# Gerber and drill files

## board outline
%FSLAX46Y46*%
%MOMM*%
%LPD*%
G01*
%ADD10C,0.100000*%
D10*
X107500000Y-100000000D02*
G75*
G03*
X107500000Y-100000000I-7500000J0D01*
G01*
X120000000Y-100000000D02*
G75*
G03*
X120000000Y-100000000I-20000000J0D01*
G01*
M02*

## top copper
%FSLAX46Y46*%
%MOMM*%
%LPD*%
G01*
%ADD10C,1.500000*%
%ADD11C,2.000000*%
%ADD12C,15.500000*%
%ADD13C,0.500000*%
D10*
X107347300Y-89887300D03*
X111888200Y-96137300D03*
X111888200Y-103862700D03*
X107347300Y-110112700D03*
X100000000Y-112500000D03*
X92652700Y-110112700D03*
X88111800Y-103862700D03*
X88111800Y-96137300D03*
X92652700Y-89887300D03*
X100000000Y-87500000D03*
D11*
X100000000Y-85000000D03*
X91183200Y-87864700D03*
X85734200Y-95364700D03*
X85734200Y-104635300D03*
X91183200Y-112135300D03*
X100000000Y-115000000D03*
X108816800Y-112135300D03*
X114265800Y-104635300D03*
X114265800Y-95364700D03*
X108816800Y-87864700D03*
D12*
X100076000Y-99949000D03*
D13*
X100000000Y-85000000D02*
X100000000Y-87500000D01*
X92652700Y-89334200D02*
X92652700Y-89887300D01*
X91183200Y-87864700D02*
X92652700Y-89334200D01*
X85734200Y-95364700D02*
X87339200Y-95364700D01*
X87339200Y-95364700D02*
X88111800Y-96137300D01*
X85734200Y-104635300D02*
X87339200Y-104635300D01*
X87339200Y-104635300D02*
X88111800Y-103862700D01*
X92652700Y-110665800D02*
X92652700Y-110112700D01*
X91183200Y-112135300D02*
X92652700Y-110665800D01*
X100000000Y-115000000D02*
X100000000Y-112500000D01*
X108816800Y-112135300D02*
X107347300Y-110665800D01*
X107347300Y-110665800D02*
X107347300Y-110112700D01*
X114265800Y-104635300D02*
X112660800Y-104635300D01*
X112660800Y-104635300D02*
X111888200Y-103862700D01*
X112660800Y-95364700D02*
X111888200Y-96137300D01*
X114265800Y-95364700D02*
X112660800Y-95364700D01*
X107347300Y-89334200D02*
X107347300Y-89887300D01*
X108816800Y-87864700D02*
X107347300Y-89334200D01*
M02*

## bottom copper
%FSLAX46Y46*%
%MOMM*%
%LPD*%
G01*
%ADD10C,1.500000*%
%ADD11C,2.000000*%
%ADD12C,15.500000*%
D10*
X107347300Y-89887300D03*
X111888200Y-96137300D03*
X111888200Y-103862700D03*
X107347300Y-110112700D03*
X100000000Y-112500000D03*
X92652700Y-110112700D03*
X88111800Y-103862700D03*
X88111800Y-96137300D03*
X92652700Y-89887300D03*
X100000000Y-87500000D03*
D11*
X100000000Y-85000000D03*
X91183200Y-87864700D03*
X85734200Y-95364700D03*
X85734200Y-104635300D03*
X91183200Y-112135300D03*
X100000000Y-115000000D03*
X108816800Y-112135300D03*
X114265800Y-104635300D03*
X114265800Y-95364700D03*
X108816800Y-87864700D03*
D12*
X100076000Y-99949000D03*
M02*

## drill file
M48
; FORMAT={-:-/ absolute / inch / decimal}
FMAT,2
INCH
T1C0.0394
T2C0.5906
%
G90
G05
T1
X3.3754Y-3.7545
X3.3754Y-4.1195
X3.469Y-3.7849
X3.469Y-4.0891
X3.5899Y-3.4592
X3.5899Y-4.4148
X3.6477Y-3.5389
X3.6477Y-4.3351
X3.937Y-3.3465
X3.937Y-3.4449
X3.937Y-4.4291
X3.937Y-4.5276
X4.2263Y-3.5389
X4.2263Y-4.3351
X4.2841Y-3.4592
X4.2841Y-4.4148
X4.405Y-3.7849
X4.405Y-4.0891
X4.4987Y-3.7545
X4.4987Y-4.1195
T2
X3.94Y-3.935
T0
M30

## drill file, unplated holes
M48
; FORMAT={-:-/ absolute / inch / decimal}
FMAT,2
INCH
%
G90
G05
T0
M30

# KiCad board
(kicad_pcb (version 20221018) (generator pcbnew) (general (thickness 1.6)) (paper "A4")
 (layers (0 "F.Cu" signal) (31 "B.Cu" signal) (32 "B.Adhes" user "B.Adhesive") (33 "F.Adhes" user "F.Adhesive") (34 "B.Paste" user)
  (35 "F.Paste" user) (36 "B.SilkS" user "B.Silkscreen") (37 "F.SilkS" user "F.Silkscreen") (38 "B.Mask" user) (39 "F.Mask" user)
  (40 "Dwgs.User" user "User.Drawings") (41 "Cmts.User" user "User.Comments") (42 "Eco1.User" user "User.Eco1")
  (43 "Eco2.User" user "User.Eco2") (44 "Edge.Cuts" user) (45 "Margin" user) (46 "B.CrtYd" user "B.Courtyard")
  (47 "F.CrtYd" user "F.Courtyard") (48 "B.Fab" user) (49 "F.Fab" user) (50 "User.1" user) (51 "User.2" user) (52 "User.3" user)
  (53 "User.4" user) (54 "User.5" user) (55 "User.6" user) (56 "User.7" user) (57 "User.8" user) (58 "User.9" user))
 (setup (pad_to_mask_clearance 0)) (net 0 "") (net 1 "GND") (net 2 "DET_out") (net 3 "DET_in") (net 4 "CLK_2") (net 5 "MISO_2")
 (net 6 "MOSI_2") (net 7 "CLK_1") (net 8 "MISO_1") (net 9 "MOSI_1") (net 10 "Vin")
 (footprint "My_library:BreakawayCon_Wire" (layer "B.Cu") (at 100 100)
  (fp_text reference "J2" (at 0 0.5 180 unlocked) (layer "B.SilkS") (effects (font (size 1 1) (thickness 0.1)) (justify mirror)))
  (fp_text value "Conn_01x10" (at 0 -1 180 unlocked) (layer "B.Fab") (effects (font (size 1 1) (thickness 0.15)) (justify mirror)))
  (pad "1" thru_hole circle (at 0 -12.5) (size 1.5 1.5) (drill 1) (layers "*.Cu" "*.Mask") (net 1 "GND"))
  (pad "2" thru_hole circle (at -7.3473 -10.1127) (size 1.5 1.5) (drill 1) (layers "*.Cu" "*.Mask") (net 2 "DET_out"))
  (pad "3" thru_hole circle (at -11.8882 -3.8627) (size 1.5 1.5) (drill 1) (layers "*.Cu" "*.Mask") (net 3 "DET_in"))
  (pad "4" thru_hole circle (at -11.8882 3.8627) (size 1.5 1.5) (drill 1) (layers "*.Cu" "*.Mask") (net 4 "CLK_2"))
  (pad "5" thru_hole circle (at -7.3473 10.1127) (size 1.5 1.5) (drill 1) (layers "*.Cu" "*.Mask") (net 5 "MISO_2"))
  (pad "6" thru_hole circle (at 0 12.5) (size 1.5 1.5) (drill 1) (layers "*.Cu" "*.Mask") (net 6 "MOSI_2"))
  (pad "7" thru_hole circle (at 7.3473 10.1127) (size 1.5 1.5) (drill 1) (layers "*.Cu" "*.Mask") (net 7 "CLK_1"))
  (pad "8" thru_hole circle (at 11.8882 3.8627) (size 1.5 1.5) (drill 1) (layers "*.Cu" "*.Mask") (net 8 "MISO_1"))
  (pad "9" thru_hole circle (at 11.8882 -3.8627) (size 1.5 1.5) (drill 1) (layers "*.Cu" "*.Mask") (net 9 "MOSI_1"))
  (pad "10" thru_hole circle (at 7.3473 -10.1127) (size 1.5 1.5) (drill 1) (layers "*.Cu" "*.Mask") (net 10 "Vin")))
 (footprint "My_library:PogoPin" (layer "B.Cu") (at 100 100)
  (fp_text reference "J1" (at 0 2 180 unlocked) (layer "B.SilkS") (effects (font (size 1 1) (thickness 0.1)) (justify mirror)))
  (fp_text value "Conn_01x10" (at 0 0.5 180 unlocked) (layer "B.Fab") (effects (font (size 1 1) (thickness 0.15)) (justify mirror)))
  (pad "1" thru_hole circle (at 0 -15) (size 2 2) (drill 1) (layers "*.Cu" "*.Mask") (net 1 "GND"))
  (pad "2" thru_hole circle (at -8.8168 -12.1353) (size 2 2) (drill 1) (layers "*.Cu" "*.Mask") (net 2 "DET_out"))
  (pad "3" thru_hole circle (at -14.2658 -4.6353) (size 2 2) (drill 1) (layers "*.Cu" "*.Mask") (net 3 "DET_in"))
  (pad "4" thru_hole circle (at -14.2658 4.6353) (size 2 2) (drill 1) (layers "*.Cu" "*.Mask") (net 4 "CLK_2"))
  (pad "5" thru_hole circle (at -8.8168 12.1353) (size 2 2) (drill 1) (layers "*.Cu" "*.Mask") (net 5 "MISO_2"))
  (pad "6" thru_hole circle (at 0 15) (size 2 2) (drill 1) (layers "*.Cu" "*.Mask") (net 6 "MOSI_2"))
  (pad "7" thru_hole circle (at 8.8168 12.1353) (size 2 2) (drill 1) (layers "*.Cu" "*.Mask") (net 7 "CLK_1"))
  (pad "8" thru_hole circle (at 14.2658 4.6353) (size 2 2) (drill 1) (layers "*.Cu" "*.Mask") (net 8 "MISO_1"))
  (pad "9" thru_hole circle (at 14.2658 -4.6353) (size 2 2) (drill 1) (layers "*.Cu" "*.Mask") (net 9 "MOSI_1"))
  (pad "10" thru_hole circle (at 8.8168 -12.1353) (size 2 2) (drill 1) (layers "*.Cu" "*.Mask") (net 10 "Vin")))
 (gr_circle (center 100 100) (end 107.5 100) (stroke (width 0.1) (type default)) (fill none) (layer "Edge.Cuts"))
 (gr_circle (center 100 100) (end 120 100) (stroke (width 0.1) (type default)) (fill none) (layer "Edge.Cuts"))
 (via (at 100.076 99.949) (size 15.5) (drill 15) (layers "F.Cu" "B.Cu") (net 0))
 (segment (start 100 85) (end 100 87.5) (width 0.5) (layer "F.Cu") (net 1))
 (segment (start 92.6527 89.3342) (end 92.6527 89.8873) (width 0.5) (layer "F.Cu") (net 2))
 (segment (start 91.1832 87.8647) (end 92.6527 89.3342) (width 0.5) (layer "F.Cu") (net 2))
 (segment (start 85.7342 95.3647) (end 87.3392 95.3647) (width 0.5) (layer "F.Cu") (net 3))
 (segment (start 87.3392 95.3647) (end 88.1118 96.1373) (width 0.5) (layer "F.Cu") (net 3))
 (segment (start 85.7342 104.6353) (end 87.3392 104.6353) (width 0.5) (layer "F.Cu") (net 4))
 (segment (start 87.3392 104.6353) (end 88.1118 103.8627) (width 0.5) (layer "F.Cu") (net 4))
 (segment (start 92.6527 110.6658) (end 92.6527 110.1127) (width 0.5) (layer "F.Cu") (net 5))
 (segment (start 91.1832 112.1353) (end 92.6527 110.6658) (width 0.5) (layer "F.Cu") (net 5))
 (segment (start 100 115) (end 100 112.5) (width 0.5) (layer "F.Cu") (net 6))
 (segment (start 108.8168 112.1353) (end 107.3473 110.6658) (width 0.5) (layer "F.Cu") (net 7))
 (segment (start 107.3473 110.6658) (end 107.3473 110.1127) (width 0.5) (layer "F.Cu") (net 7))
 (segment (start 114.2658 104.6353) (end 112.6608 104.6353) (width 0.5) (layer "F.Cu") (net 8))
 (segment (start 112.6608 104.6353) (end 111.8882 103.8627) (width 0.5) (layer "F.Cu") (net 8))
 (segment (start 112.6608 95.3647) (end 111.8882 96.1373) (width 0.5) (layer "F.Cu") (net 9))
 (segment (start 114.2658 95.3647) (end 112.6608 95.3647) (width 0.5) (layer "F.Cu") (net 9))
 (segment (start 107.3473 89.3342) (end 107.3473 89.8873) (width 0.5) (layer "F.Cu") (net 10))
 (segment (start 108.8168 87.8647) (end 107.3473 89.3342) (width 0.5) (layer "F.Cu") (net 10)))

